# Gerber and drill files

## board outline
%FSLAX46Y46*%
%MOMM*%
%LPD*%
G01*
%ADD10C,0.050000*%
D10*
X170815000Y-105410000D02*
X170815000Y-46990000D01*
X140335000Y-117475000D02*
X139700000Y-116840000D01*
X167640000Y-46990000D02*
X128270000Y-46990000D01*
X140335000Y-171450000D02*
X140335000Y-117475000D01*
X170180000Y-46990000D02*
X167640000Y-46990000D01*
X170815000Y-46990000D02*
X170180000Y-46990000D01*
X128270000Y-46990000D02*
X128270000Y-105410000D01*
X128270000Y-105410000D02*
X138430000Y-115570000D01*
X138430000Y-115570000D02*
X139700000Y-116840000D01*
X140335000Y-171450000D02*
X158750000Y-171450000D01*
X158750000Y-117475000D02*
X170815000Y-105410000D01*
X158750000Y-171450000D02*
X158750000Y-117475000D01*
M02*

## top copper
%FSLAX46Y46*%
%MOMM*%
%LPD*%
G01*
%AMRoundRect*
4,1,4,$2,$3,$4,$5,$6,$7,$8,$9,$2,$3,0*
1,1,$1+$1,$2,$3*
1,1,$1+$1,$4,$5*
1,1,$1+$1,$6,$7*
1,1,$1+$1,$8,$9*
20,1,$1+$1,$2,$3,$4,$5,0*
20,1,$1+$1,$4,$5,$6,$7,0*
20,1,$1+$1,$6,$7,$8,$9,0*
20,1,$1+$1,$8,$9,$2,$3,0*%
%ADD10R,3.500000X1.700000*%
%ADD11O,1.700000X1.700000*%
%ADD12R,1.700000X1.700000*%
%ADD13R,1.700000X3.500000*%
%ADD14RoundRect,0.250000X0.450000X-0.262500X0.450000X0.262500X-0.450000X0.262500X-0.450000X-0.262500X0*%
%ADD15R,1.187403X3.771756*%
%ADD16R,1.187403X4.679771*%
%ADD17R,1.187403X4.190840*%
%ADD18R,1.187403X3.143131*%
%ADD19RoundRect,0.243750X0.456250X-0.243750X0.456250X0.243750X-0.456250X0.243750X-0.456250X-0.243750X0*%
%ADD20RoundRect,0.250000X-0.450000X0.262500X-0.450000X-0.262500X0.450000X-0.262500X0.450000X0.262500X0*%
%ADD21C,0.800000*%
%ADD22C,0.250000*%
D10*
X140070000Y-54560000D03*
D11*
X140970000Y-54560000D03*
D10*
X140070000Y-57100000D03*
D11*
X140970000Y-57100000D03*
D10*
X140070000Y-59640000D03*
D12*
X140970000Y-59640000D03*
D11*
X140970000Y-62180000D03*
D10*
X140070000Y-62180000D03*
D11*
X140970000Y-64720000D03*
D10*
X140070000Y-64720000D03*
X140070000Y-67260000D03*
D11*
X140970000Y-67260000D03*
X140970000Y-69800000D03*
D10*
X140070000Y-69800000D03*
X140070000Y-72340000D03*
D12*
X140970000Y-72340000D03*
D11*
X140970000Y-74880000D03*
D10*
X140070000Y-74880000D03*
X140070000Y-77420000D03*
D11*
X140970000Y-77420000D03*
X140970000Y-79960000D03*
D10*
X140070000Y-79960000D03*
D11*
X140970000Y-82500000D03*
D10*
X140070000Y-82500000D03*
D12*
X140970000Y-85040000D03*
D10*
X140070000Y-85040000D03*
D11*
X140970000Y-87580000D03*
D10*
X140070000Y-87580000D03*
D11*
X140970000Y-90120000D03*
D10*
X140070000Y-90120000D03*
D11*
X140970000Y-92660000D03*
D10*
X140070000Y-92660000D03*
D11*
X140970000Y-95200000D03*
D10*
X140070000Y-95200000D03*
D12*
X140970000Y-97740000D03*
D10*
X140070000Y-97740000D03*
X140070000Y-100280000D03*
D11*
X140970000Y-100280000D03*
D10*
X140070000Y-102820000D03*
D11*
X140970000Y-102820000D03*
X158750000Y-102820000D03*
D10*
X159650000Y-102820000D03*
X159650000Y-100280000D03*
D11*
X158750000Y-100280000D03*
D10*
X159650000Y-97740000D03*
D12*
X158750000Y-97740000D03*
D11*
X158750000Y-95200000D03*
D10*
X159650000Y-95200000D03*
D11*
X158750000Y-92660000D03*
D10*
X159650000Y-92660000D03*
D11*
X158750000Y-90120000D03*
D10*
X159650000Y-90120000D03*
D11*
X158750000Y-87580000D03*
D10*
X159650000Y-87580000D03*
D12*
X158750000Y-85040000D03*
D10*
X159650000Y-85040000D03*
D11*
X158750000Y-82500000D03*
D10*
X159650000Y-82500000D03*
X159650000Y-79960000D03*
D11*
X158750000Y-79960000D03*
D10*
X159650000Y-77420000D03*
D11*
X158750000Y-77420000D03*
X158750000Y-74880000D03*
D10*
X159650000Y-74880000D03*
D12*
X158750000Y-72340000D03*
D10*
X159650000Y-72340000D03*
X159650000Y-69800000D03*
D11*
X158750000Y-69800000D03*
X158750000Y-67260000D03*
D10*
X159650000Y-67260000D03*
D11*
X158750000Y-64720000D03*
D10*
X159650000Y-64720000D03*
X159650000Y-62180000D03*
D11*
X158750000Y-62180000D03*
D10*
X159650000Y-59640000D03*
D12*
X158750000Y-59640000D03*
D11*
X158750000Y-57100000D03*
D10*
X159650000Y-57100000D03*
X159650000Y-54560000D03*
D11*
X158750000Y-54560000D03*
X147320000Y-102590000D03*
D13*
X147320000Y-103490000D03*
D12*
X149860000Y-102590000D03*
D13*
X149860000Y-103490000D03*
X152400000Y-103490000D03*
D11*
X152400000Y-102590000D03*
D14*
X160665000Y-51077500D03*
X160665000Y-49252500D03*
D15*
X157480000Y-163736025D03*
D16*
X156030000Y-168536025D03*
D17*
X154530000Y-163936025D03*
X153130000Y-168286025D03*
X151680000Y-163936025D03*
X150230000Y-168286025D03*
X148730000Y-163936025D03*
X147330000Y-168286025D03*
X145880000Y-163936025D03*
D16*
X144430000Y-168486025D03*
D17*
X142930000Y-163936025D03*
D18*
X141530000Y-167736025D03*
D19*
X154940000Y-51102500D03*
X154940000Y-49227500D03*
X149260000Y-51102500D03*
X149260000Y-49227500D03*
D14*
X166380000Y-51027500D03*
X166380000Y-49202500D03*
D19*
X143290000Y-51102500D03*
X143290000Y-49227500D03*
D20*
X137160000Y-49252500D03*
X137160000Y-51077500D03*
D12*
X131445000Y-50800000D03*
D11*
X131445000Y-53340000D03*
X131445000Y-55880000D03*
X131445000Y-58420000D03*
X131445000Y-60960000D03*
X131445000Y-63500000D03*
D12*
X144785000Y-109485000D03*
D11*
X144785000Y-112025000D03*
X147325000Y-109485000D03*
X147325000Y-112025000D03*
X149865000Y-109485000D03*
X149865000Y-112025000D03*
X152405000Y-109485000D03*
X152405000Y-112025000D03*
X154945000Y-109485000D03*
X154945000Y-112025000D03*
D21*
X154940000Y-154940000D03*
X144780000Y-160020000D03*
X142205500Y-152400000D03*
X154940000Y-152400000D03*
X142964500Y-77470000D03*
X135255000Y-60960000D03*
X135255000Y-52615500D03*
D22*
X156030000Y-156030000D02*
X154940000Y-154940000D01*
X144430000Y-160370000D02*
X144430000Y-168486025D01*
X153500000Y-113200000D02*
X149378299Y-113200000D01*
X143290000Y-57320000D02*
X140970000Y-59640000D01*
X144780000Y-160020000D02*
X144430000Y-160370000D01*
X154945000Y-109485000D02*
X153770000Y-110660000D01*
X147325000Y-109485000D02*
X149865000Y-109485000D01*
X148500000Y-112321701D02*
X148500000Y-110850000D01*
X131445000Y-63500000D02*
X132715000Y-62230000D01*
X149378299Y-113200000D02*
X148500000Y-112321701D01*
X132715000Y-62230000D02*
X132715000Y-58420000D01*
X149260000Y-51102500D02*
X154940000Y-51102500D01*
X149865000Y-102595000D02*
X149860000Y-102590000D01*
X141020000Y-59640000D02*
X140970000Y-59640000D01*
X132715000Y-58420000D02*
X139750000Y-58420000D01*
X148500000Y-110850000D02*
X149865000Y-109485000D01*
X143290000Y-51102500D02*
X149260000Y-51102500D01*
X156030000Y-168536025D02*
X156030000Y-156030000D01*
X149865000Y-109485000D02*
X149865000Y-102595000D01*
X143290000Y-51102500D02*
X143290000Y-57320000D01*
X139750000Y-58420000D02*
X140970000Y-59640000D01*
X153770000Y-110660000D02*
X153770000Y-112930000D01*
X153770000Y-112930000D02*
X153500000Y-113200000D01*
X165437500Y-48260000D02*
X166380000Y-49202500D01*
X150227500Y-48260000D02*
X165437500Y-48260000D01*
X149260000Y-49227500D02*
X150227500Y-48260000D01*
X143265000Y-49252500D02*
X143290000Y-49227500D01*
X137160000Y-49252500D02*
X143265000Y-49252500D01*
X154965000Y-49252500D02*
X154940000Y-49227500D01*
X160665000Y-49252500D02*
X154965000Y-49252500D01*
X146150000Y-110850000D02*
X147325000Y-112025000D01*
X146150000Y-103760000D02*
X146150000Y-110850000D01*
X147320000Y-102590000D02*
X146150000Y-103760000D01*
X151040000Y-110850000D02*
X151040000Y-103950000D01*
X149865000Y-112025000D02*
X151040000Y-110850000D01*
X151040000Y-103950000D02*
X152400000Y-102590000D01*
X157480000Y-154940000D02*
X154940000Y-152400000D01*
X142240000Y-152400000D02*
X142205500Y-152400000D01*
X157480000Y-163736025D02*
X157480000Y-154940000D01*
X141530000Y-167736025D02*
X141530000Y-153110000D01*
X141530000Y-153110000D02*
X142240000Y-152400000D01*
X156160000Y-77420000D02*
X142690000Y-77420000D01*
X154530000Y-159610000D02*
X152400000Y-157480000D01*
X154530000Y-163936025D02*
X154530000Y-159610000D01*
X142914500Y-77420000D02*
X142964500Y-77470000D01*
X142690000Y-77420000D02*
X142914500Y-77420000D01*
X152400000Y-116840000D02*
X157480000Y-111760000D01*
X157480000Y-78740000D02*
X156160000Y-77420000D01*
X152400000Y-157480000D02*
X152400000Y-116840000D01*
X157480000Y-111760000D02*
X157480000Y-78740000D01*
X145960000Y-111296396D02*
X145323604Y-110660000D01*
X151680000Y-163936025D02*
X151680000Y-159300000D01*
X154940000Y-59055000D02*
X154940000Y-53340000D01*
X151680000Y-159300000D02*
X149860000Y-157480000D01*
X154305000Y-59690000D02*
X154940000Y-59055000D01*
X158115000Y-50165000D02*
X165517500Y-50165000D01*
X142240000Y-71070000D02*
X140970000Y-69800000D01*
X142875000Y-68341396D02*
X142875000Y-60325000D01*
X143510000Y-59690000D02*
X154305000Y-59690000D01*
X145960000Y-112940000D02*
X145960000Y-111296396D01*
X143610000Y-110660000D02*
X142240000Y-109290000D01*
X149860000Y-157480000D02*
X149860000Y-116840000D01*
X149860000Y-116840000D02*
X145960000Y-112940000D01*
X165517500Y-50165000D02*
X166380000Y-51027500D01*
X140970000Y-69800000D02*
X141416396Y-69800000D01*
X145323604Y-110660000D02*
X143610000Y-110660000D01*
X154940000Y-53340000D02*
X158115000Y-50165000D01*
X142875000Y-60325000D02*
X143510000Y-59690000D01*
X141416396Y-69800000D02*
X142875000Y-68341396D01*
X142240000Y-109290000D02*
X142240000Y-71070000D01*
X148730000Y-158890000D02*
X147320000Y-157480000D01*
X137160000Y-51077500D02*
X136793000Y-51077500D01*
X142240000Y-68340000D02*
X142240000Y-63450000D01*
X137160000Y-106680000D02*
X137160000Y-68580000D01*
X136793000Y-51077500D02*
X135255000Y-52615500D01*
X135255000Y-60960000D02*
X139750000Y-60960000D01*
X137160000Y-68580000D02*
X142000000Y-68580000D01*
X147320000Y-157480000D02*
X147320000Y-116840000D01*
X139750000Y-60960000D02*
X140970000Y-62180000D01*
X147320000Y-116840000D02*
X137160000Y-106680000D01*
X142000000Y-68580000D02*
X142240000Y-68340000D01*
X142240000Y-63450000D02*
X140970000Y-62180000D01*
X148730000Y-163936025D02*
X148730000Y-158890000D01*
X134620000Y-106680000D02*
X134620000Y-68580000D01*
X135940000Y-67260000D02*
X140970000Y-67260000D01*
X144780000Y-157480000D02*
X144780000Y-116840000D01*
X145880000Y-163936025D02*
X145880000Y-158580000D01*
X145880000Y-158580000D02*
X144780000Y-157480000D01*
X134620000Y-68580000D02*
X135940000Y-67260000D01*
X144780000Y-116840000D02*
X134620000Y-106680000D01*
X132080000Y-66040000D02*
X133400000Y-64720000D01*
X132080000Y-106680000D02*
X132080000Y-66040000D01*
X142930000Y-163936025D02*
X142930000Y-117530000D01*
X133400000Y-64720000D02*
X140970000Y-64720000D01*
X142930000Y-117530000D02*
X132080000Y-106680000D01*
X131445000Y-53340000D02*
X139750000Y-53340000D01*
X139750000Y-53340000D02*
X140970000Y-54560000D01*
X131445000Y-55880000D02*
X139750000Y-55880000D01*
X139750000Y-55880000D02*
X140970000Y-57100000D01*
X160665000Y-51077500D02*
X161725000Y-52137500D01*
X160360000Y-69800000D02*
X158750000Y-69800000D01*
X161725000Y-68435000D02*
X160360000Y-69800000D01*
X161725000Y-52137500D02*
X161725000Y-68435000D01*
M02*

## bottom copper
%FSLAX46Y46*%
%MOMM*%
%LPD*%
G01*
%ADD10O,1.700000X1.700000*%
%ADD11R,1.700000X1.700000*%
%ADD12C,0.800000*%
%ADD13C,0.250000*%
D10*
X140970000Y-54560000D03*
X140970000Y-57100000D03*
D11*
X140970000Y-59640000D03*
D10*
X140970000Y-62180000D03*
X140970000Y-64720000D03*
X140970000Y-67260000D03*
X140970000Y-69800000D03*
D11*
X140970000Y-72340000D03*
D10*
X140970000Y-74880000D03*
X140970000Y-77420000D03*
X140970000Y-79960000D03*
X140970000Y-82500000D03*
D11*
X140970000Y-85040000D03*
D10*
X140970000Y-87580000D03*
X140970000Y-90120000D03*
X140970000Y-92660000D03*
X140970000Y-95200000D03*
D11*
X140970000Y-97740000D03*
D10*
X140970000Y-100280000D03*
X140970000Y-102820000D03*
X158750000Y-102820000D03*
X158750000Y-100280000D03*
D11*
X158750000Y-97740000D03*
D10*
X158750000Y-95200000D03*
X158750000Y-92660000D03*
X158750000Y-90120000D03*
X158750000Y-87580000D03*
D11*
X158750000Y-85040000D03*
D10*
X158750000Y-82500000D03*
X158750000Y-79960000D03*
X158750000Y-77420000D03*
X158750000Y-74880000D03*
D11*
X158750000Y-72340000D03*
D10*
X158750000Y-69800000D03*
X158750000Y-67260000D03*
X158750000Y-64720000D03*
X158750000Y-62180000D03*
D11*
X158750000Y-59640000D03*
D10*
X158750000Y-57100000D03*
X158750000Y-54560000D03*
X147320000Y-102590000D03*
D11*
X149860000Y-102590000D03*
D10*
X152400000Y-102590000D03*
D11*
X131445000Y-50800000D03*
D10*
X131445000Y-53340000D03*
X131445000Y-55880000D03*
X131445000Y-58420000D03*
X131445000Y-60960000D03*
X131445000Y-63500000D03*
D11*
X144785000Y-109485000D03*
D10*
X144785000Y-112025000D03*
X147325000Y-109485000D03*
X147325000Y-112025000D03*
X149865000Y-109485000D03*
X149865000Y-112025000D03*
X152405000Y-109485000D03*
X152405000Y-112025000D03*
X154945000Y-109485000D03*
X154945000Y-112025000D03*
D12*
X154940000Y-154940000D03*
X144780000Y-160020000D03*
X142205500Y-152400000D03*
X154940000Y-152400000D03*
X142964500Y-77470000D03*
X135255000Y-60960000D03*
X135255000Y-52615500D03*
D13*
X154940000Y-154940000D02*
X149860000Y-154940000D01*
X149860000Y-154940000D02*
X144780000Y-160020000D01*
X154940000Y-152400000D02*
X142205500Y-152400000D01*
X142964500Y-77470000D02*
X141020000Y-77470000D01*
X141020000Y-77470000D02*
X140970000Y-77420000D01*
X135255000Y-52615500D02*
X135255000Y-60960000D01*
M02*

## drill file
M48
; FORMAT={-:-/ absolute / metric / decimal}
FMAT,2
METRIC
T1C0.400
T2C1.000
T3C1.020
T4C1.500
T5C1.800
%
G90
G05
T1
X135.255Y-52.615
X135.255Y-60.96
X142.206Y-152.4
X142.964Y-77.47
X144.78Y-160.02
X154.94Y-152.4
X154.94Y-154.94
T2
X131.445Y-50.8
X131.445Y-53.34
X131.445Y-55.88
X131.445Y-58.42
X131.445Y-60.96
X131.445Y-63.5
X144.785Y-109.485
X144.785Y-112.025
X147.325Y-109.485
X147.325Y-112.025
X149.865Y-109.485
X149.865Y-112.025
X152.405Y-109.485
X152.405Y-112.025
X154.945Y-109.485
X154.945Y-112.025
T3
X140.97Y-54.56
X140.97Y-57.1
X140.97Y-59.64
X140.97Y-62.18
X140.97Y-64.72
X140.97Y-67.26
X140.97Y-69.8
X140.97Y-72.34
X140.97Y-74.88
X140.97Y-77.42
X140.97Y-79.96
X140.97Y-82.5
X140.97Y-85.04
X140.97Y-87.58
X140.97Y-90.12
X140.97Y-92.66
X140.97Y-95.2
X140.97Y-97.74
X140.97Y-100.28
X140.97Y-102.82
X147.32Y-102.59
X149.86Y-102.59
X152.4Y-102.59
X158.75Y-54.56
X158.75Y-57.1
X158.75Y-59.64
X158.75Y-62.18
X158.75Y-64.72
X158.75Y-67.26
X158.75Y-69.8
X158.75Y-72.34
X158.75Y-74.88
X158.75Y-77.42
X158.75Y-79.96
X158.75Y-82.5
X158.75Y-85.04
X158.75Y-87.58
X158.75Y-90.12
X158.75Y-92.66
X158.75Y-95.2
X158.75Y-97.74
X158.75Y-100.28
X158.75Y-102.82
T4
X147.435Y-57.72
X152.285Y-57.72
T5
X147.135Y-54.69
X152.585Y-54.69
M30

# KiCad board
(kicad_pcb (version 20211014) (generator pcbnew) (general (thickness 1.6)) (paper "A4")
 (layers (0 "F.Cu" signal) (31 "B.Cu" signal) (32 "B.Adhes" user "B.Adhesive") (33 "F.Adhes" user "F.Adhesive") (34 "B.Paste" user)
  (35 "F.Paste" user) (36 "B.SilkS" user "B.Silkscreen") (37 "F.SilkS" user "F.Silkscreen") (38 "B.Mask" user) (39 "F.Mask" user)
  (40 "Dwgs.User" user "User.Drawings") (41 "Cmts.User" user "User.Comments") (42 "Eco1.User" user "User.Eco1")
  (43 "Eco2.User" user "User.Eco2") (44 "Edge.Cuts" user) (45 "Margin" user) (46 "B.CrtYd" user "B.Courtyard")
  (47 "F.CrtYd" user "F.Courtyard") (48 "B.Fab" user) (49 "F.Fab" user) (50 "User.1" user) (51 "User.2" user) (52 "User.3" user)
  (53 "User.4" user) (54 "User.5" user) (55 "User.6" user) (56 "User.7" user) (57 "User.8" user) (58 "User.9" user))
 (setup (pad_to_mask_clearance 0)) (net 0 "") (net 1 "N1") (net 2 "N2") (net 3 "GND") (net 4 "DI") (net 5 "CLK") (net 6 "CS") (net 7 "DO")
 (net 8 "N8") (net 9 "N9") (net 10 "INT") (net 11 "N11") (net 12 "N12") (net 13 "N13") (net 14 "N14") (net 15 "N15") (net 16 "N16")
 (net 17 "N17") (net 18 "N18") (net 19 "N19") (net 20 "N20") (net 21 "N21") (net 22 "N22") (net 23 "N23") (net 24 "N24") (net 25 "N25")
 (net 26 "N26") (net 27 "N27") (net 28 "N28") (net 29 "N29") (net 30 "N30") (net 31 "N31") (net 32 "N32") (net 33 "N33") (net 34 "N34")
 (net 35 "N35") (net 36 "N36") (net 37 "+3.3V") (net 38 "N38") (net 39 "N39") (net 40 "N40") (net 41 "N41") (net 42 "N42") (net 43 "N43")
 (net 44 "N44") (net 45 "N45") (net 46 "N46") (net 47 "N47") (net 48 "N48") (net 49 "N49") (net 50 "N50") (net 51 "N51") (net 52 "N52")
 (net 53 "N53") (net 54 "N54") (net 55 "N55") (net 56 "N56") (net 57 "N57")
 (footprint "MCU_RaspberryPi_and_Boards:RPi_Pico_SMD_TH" (layer "F.Cu") (at 149.86 78.69)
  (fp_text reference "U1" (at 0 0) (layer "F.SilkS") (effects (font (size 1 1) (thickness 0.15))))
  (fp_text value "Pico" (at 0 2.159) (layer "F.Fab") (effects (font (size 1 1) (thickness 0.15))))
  (pad "" np_thru_hole oval (at -2.725 -24) (size 1.8 1.8) (drill 1.8) (layers *.Cu *.Mask))
  (pad "" np_thru_hole oval (at 2.725 -24) (size 1.8 1.8) (drill 1.8) (layers *.Cu *.Mask))
  (pad "" np_thru_hole oval (at 2.425 -20.97) (size 1.5 1.5) (drill 1.5) (layers *.Cu *.Mask))
  (pad "" np_thru_hole oval (at -2.425 -20.97) (size 1.5 1.5) (drill 1.5) (layers *.Cu *.Mask))
  (pad "1" smd rect (at -8.89 -24.13) (size 3.5 1.7) (drill (offset -0.9 0)) (layers "F.Cu" "F.Mask") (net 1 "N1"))
  (pad "1" thru_hole oval (at -8.89 -24.13) (size 1.7 1.7) (drill 1.02) (layers *.Cu *.Mask) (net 1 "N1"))
  (pad "2" smd rect (at -8.89 -21.59) (size 3.5 1.7) (drill (offset -0.9 0)) (layers "F.Cu" "F.Mask") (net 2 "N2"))
  (pad "2" thru_hole oval (at -8.89 -21.59) (size 1.7 1.7) (drill 1.02) (layers *.Cu *.Mask) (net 2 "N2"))
  (pad "3" smd rect (at -8.89 -19.05) (size 3.5 1.7) (drill (offset -0.9 0)) (layers "F.Cu" "F.Mask") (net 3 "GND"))
  (pad "3" thru_hole rect (at -8.89 -19.05) (size 1.7 1.7) (drill 1.02) (layers *.Cu *.Mask) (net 3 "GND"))
  (pad "4" thru_hole oval (at -8.89 -16.51) (size 1.7 1.7) (drill 1.02) (layers *.Cu *.Mask) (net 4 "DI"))
  (pad "4" smd rect (at -8.89 -16.51) (size 3.5 1.7) (drill (offset -0.9 0)) (layers "F.Cu" "F.Mask") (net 4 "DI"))
  (pad "5" thru_hole oval (at -8.89 -13.97) (size 1.7 1.7) (drill 1.02) (layers *.Cu *.Mask) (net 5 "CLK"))
  (pad "5" smd rect (at -8.89 -13.97) (size 3.5 1.7) (drill (offset -0.9 0)) (layers "F.Cu" "F.Mask") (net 5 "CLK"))
  (pad "6" smd rect (at -8.89 -11.43) (size 3.5 1.7) (drill (offset -0.9 0)) (layers "F.Cu" "F.Mask") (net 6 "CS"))
  (pad "6" thru_hole oval (at -8.89 -11.43) (size 1.7 1.7) (drill 1.02) (layers *.Cu *.Mask) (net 6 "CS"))
  (pad "7" thru_hole oval (at -8.89 -8.89) (size 1.7 1.7) (drill 1.02) (layers *.Cu *.Mask) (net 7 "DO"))
  (pad "7" smd rect (at -8.89 -8.89) (size 3.5 1.7) (drill (offset -0.9 0)) (layers "F.Cu" "F.Mask") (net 7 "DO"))
  (pad "8" smd rect (at -8.89 -6.35) (size 3.5 1.7) (drill (offset -0.9 0)) (layers "F.Cu" "F.Mask") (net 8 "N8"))
  (pad "8" thru_hole rect (at -8.89 -6.35) (size 1.7 1.7) (drill 1.02) (layers *.Cu *.Mask) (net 8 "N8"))
  (pad "9" thru_hole oval (at -8.89 -3.81) (size 1.7 1.7) (drill 1.02) (layers *.Cu *.Mask) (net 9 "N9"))
  (pad "9" smd rect (at -8.89 -3.81) (size 3.5 1.7) (drill (offset -0.9 0)) (layers "F.Cu" "F.Mask") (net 9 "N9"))
  (pad "10" smd rect (at -8.89 -1.27) (size 3.5 1.7) (drill (offset -0.9 0)) (layers "F.Cu" "F.Mask") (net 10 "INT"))
  (pad "10" thru_hole oval (at -8.89 -1.27) (size 1.7 1.7) (drill 1.02) (layers *.Cu *.Mask) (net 10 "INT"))
  (pad "11" thru_hole oval (at -8.89 1.27) (size 1.7 1.7) (drill 1.02) (layers *.Cu *.Mask) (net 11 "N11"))
  (pad "11" smd rect (at -8.89 1.27) (size 3.5 1.7) (drill (offset -0.9 0)) (layers "F.Cu" "F.Mask") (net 11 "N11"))
  (pad "12" thru_hole oval (at -8.89 3.81) (size 1.7 1.7) (drill 1.02) (layers *.Cu *.Mask) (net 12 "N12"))
  (pad "12" smd rect (at -8.89 3.81) (size 3.5 1.7) (drill (offset -0.9 0)) (layers "F.Cu" "F.Mask") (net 12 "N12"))
  (pad "13" thru_hole rect (at -8.89 6.35) (size 1.7 1.7) (drill 1.02) (layers *.Cu *.Mask) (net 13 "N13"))
  (pad "13" smd rect (at -8.89 6.35) (size 3.5 1.7) (drill (offset -0.9 0)) (layers "F.Cu" "F.Mask") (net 13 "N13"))
  (pad "14" thru_hole oval (at -8.89 8.89) (size 1.7 1.7) (drill 1.02) (layers *.Cu *.Mask) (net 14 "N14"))
  (pad "14" smd rect (at -8.89 8.89) (size 3.5 1.7) (drill (offset -0.9 0)) (layers "F.Cu" "F.Mask") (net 14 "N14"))
  (pad "15" thru_hole oval (at -8.89 11.43) (size 1.7 1.7) (drill 1.02) (layers *.Cu *.Mask) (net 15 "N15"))
  (pad "15" smd rect (at -8.89 11.43) (size 3.5 1.7) (drill (offset -0.9 0)) (layers "F.Cu" "F.Mask") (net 15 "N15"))
  (pad "16" thru_hole oval (at -8.89 13.97) (size 1.7 1.7) (drill 1.02) (layers *.Cu *.Mask) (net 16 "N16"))
  (pad "16" smd rect (at -8.89 13.97) (size 3.5 1.7) (drill (offset -0.9 0)) (layers "F.Cu" "F.Mask") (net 16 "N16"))
  (pad "17" thru_hole oval (at -8.89 16.51) (size 1.7 1.7) (drill 1.02) (layers *.Cu *.Mask) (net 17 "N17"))
  (pad "17" smd rect (at -8.89 16.51) (size 3.5 1.7) (drill (offset -0.9 0)) (layers "F.Cu" "F.Mask") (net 17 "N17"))
  (pad "18" thru_hole rect (at -8.89 19.05) (size 1.7 1.7) (drill 1.02) (layers *.Cu *.Mask) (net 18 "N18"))
  (pad "18" smd rect (at -8.89 19.05) (size 3.5 1.7) (drill (offset -0.9 0)) (layers "F.Cu" "F.Mask") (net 18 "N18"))
  (pad "19" smd rect (at -8.89 21.59) (size 3.5 1.7) (drill (offset -0.9 0)) (layers "F.Cu" "F.Mask") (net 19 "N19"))
  (pad "19" thru_hole oval (at -8.89 21.59) (size 1.7 1.7) (drill 1.02) (layers *.Cu *.Mask) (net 19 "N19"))
  (pad "20" smd rect (at -8.89 24.13) (size 3.5 1.7) (drill (offset -0.9 0)) (layers "F.Cu" "F.Mask") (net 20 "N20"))
  (pad "20" thru_hole oval (at -8.89 24.13) (size 1.7 1.7) (drill 1.02) (layers *.Cu *.Mask) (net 20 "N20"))
  (pad "21" thru_hole oval (at 8.89 24.13) (size 1.7 1.7) (drill 1.02) (layers *.Cu *.Mask) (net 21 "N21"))
  (pad "21" smd rect (at 8.89 24.13) (size 3.5 1.7) (drill (offset 0.9 0)) (layers "F.Cu" "F.Mask") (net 21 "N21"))
  (pad "22" smd rect (at 8.89 21.59) (size 3.5 1.7) (drill (offset 0.9 0)) (layers "F.Cu" "F.Mask") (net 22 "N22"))
  (pad "22" thru_hole oval (at 8.89 21.59) (size 1.7 1.7) (drill 1.02) (layers *.Cu *.Mask) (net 22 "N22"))
  (pad "23" smd rect (at 8.89 19.05) (size 3.5 1.7) (drill (offset 0.9 0)) (layers "F.Cu" "F.Mask") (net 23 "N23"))
  (pad "23" thru_hole rect (at 8.89 19.05) (size 1.7 1.7) (drill 1.02) (layers *.Cu *.Mask) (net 23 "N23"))
  (pad "24" thru_hole oval (at 8.89 16.51) (size 1.7 1.7) (drill 1.02) (layers *.Cu *.Mask) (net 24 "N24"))
  (pad "24" smd rect (at 8.89 16.51) (size 3.5 1.7) (drill (offset 0.9 0)) (layers "F.Cu" "F.Mask") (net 24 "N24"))
  (pad "25" thru_hole oval (at 8.89 13.97) (size 1.7 1.7) (drill 1.02) (layers *.Cu *.Mask) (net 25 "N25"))
  (pad "25" smd rect (at 8.89 13.97) (size 3.5 1.7) (drill (offset 0.9 0)) (layers "F.Cu" "F.Mask") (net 25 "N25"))
  (pad "26" thru_hole oval (at 8.89 11.43) (size 1.7 1.7) (drill 1.02) (layers *.Cu *.Mask) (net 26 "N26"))
  (pad "26" smd rect (at 8.89 11.43) (size 3.5 1.7) (drill (offset 0.9 0)) (layers "F.Cu" "F.Mask") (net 26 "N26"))
  (pad "27" thru_hole oval (at 8.89 8.89) (size 1.7 1.7) (drill 1.02) (layers *.Cu *.Mask) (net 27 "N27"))
  (pad "27" smd rect (at 8.89 8.89) (size 3.5 1.7) (drill (offset 0.9 0)) (layers "F.Cu" "F.Mask") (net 27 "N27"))
  (pad "28" thru_hole rect (at 8.89 6.35) (size 1.7 1.7) (drill 1.02) (layers *.Cu *.Mask) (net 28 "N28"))
  (pad "28" smd rect (at 8.89 6.35) (size 3.5 1.7) (drill (offset 0.9 0)) (layers "F.Cu" "F.Mask") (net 28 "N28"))
  (pad "29" thru_hole oval (at 8.89 3.81) (size 1.7 1.7) (drill 1.02) (layers *.Cu *.Mask) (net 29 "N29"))
  (pad "29" smd rect (at 8.89 3.81) (size 3.5 1.7) (drill (offset 0.9 0)) (layers "F.Cu" "F.Mask") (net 29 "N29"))
  (pad "30" smd rect (at 8.89 1.27) (size 3.5 1.7) (drill (offset 0.9 0)) (layers "F.Cu" "F.Mask") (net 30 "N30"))
  (pad "30" thru_hole oval (at 8.89 1.27) (size 1.7 1.7) (drill 1.02) (layers *.Cu *.Mask) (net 30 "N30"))
  (pad "31" smd rect (at 8.89 -1.27) (size 3.5 1.7) (drill (offset 0.9 0)) (layers "F.Cu" "F.Mask") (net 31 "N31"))
  (pad "31" thru_hole oval (at 8.89 -1.27) (size 1.7 1.7) (drill 1.02) (layers *.Cu *.Mask) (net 31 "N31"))
  (pad "32" thru_hole oval (at 8.89 -3.81) (size 1.7 1.7) (drill 1.02) (layers *.Cu *.Mask) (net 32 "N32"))
  (pad "32" smd rect (at 8.89 -3.81) (size 3.5 1.7) (drill (offset 0.9 0)) (layers "F.Cu" "F.Mask") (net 32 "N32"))
  (pad "33" thru_hole rect (at 8.89 -6.35) (size 1.7 1.7) (drill 1.02) (layers *.Cu *.Mask) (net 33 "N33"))
  (pad "33" smd rect (at 8.89 -6.35) (size 3.5 1.7) (drill (offset 0.9 0)) (layers "F.Cu" "F.Mask") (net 33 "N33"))
  (pad "34" smd rect (at 8.89 -8.89) (size 3.5 1.7) (drill (offset 0.9 0)) (layers "F.Cu" "F.Mask") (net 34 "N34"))
  (pad "34" thru_hole oval (at 8.89 -8.89) (size 1.7 1.7) (drill 1.02) (layers *.Cu *.Mask) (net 34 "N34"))
  (pad "35" thru_hole oval (at 8.89 -11.43) (size 1.7 1.7) (drill 1.02) (layers *.Cu *.Mask) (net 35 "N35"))
  (pad "35" smd rect (at 8.89 -11.43) (size 3.5 1.7) (drill (offset 0.9 0)) (layers "F.Cu" "F.Mask") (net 35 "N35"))
  (pad "36" thru_hole oval (at 8.89 -13.97) (size 1.7 1.7) (drill 1.02) (layers *.Cu *.Mask) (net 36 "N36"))
  (pad "36" smd rect (at 8.89 -13.97) (size 3.5 1.7) (drill (offset 0.9 0)) (layers "F.Cu" "F.Mask") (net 36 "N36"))
  (pad "37" smd rect (at 8.89 -16.51) (size 3.5 1.7) (drill (offset 0.9 0)) (layers "F.Cu" "F.Mask") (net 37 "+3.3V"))
  (pad "37" thru_hole oval (at 8.89 -16.51) (size 1.7 1.7) (drill 1.02) (layers *.Cu *.Mask) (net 37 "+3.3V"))
  (pad "38" smd rect (at 8.89 -19.05) (size 3.5 1.7) (drill (offset 0.9 0)) (layers "F.Cu" "F.Mask") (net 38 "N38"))
  (pad "38" thru_hole rect (at 8.89 -19.05) (size 1.7 1.7) (drill 1.02) (layers *.Cu *.Mask) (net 38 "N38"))
  (pad "39" thru_hole oval (at 8.89 -21.59) (size 1.7 1.7) (drill 1.02) (layers *.Cu *.Mask) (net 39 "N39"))
  (pad "39" smd rect (at 8.89 -21.59) (size 3.5 1.7) (drill (offset 0.9 0)) (layers "F.Cu" "F.Mask") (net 39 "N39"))
  (pad "40" smd rect (at 8.89 -24.13) (size 3.5 1.7) (drill (offset 0.9 0)) (layers "F.Cu" "F.Mask") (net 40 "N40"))
  (pad "40" thru_hole oval (at 8.89 -24.13) (size 1.7 1.7) (drill 1.02) (layers *.Cu *.Mask) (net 40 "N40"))
  (pad "41" thru_hole oval (at -2.54 23.9) (size 1.7 1.7) (drill 1.02) (layers *.Cu *.Mask) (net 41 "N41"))
  (pad "41" smd rect (at -2.54 23.9 90) (size 3.5 1.7) (drill (offset -0.9 0)) (layers "F.Cu" "F.Mask") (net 41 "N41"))
  (pad "42" thru_hole rect (at 0 23.9) (size 1.7 1.7) (drill 1.02) (layers *.Cu *.Mask) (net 3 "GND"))
  (pad "42" smd rect (at 0 23.9 90) (size 3.5 1.7) (drill (offset -0.9 0)) (layers "F.Cu" "F.Mask") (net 3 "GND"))
  (pad "43" smd rect (at 2.54 23.9 90) (size 3.5 1.7) (drill (offset -0.9 0)) (layers "F.Cu" "F.Mask") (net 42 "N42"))
  (pad "43" thru_hole oval (at 2.54 23.9) (size 1.7 1.7) (drill 1.02) (layers *.Cu *.Mask) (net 42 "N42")))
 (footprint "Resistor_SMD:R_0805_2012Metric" (layer "F.Cu") (at 160.665 50.165 90)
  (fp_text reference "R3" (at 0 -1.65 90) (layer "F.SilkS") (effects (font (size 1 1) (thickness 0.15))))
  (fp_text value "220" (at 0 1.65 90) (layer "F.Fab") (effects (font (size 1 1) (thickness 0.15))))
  (pad "1" smd roundrect (at -0.9125 0 90) (size 1.025 1.4) (layers "F.Cu" "F.Paste" "F.Mask") (roundrect_rratio 0.243902439) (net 34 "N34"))
  (pad "2" smd roundrect (at 0.9125 0 90) (size 1.025 1.4) (layers "F.Cu" "F.Paste" "F.Mask") (roundrect_rratio 0.243902439) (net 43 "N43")))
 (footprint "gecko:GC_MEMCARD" (layer "F.Cu") (at 140.43 171.316025)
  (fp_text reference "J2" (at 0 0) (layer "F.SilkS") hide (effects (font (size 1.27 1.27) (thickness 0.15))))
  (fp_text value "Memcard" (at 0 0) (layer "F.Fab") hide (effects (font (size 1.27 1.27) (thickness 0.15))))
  (pad "1" smd rect (at 17.05 -7.58) (size 1.187403 3.771756) (layers "F.Cu" "F.Paste" "F.Mask") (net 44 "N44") (solder_mask_margin 0.0762))
  (pad "2" smd rect (at 15.6 -2.78) (size 1.187403 4.679771) (layers "F.Cu" "F.Paste" "F.Mask") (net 3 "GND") (solder_mask_margin 0.0762))
  (pad "3" smd rect (at 14.1 -7.38) (size 1.187403 4.19084) (layers "F.Cu" "F.Paste" "F.Mask") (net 10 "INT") (solder_mask_margin 0.0762))
  (pad "4" smd rect (at 12.7 -3.03) (size 1.187403 4.19084) (layers "F.Cu" "F.Paste" "F.Mask") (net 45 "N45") (solder_mask_margin 0.0762))
  (pad "5" smd rect (at 11.25 -7.38) (size 1.187403 4.19084) (layers "F.Cu" "F.Paste" "F.Mask") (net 7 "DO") (solder_mask_margin 0.0762))
  (pad "6" smd rect (at 9.8 -3.03) (size 1.187403 4.19084) (layers "F.Cu" "F.Paste" "F.Mask") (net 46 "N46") (solder_mask_margin 0.0762))
  (pad "7" smd rect (at 8.3 -7.38) (size 1.187403 4.19084) (layers "F.Cu" "F.Paste" "F.Mask") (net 4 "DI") (solder_mask_margin 0.0762))
  (pad "8" smd rect (at 6.9 -3.03) (size 1.187403 4.19084) (layers "F.Cu" "F.Paste" "F.Mask") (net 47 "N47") (solder_mask_margin 0.0762))
  (pad "9" smd rect (at 5.45 -7.38) (size 1.187403 4.19084) (layers "F.Cu" "F.Paste" "F.Mask") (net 6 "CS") (solder_mask_margin 0.0762))
  (pad "10" smd rect (at 4 -2.83) (size 1.187403 4.679771) (layers "F.Cu" "F.Paste" "F.Mask") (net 3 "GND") (solder_mask_margin 0.0762))
  (pad "11" smd rect (at 2.5 -7.38) (size 1.187403 4.19084) (layers "F.Cu" "F.Paste" "F.Mask") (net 5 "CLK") (solder_mask_margin 0.0762))
  (pad "12" smd rect (at 1.1 -3.58) (size 1.187403 3.143131) (layers "F.Cu" "F.Paste" "F.Mask") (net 44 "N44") (solder_mask_margin 0.0762)))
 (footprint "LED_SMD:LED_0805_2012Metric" (layer "F.Cu") (at 154.94 50.165 90)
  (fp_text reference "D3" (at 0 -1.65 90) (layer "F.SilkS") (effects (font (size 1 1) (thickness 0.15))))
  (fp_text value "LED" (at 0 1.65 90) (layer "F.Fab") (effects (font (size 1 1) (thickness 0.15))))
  (pad "1" smd roundrect (at -0.9375 0 90) (size 0.975 1.4) (layers "F.Cu" "F.Paste" "F.Mask") (roundrect_rratio 0.25) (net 3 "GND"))
  (pad "2" smd roundrect (at 0.9375 0 90) (size 0.975 1.4) (layers "F.Cu" "F.Paste" "F.Mask") (roundrect_rratio 0.25) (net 43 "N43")))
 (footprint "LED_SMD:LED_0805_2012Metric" (layer "F.Cu") (at 149.26 50.165 90)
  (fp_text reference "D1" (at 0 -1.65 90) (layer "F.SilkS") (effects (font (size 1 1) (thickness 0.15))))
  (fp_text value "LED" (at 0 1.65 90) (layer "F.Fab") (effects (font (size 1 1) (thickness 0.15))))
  (pad "1" smd roundrect (at -0.9375 0 90) (size 0.975 1.4) (layers "F.Cu" "F.Paste" "F.Mask") (roundrect_rratio 0.25) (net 3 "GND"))
  (pad "2" smd roundrect (at 0.9375 0 90) (size 0.975 1.4) (layers "F.Cu" "F.Paste" "F.Mask") (roundrect_rratio 0.25) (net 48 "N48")))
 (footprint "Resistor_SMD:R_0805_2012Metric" (layer "F.Cu") (at 166.38 50.115 90)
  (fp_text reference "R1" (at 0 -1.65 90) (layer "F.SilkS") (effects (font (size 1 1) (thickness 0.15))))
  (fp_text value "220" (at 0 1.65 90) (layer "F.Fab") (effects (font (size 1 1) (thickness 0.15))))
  (pad "1" smd roundrect (at -0.9125 0 90) (size 1.025 1.4) (layers "F.Cu" "F.Paste" "F.Mask") (roundrect_rratio 0.243902439) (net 7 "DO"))
  (pad "2" smd roundrect (at 0.9125 0 90) (size 1.025 1.4) (layers "F.Cu" "F.Paste" "F.Mask") (roundrect_rratio 0.243902439) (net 48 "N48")))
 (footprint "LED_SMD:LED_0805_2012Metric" (layer "F.Cu") (at 143.29 50.165 90)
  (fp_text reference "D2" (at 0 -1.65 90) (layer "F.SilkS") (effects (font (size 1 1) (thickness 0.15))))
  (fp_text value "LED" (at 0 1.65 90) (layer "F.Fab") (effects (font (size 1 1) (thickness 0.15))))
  (pad "1" smd roundrect (at -0.9375 0 90) (size 0.975 1.4) (layers "F.Cu" "F.Paste" "F.Mask") (roundrect_rratio 0.25) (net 3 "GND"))
  (pad "2" smd roundrect (at 0.9375 0 90) (size 0.975 1.4) (layers "F.Cu" "F.Paste" "F.Mask") (roundrect_rratio 0.25) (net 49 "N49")))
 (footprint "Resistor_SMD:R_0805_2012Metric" (layer "F.Cu") (at 137.16 50.165 -90)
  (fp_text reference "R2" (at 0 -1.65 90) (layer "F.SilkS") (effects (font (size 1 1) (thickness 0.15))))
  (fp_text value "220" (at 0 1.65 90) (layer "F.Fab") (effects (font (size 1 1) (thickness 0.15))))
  (pad "1" smd roundrect (at -0.9125 0 270) (size 1.025 1.4) (layers "F.Cu" "F.Paste" "F.Mask") (roundrect_rratio 0.243902439)
   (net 49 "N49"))
  (pad "2" smd roundrect (at 0.9125 0 270) (size 1.025 1.4) (layers "F.Cu" "F.Paste" "F.Mask") (roundrect_rratio 0.243902439) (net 4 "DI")))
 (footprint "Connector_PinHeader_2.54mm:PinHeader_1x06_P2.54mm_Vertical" (layer "B.Cu") (at 131.445 50.8 180)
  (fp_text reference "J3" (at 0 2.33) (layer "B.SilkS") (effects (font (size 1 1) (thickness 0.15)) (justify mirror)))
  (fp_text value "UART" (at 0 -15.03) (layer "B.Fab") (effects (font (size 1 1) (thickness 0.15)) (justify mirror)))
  (pad "1" thru_hole rect (at 0 0 180) (size 1.7 1.7) (drill 1) (layers *.Cu *.Mask) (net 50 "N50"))
  (pad "2" thru_hole oval (at 0 -2.54 180) (size 1.7 1.7) (drill 1) (layers *.Cu *.Mask) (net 1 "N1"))
  (pad "3" thru_hole oval (at 0 -5.08 180) (size 1.7 1.7) (drill 1) (layers *.Cu *.Mask) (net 2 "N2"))
  (pad "4" thru_hole oval (at 0 -7.62 180) (size 1.7 1.7) (drill 1) (layers *.Cu *.Mask) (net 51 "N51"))
  (pad "5" thru_hole oval (at 0 -10.16 180) (size 1.7 1.7) (drill 1) (layers *.Cu *.Mask) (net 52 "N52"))
  (pad "6" thru_hole oval (at 0 -12.7 180) (size 1.7 1.7) (drill 1) (layers *.Cu *.Mask) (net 3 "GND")))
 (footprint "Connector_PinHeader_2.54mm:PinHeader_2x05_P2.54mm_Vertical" (layer "B.Cu") (at 144.785 109.485 -90)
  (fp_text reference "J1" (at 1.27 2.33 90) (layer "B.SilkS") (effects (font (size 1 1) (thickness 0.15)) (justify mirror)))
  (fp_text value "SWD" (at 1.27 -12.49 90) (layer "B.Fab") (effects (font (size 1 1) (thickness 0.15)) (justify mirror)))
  (pad "1" thru_hole rect (at 0 0 270) (size 1.7 1.7) (drill 1) (layers *.Cu *.Mask) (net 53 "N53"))
  (pad "2" thru_hole oval (at 2.54 0 270) (size 1.7 1.7) (drill 1) (layers *.Cu *.Mask) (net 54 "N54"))
  (pad "3" thru_hole oval (at 0 -2.54 270) (size 1.7 1.7) (drill 1) (layers *.Cu *.Mask) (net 3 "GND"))
  (pad "4" thru_hole oval (at 2.54 -2.54 270) (size 1.7 1.7) (drill 1) (layers *.Cu *.Mask) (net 41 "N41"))
  (pad "5" thru_hole oval (at 0 -5.08 270) (size 1.7 1.7) (drill 1) (layers *.Cu *.Mask) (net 3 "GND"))
  (pad "6" thru_hole oval (at 2.54 -5.08 270) (size 1.7 1.7) (drill 1) (layers *.Cu *.Mask) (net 42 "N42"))
  (pad "7" thru_hole oval (at 0 -7.62 270) (size 1.7 1.7) (drill 1) (layers *.Cu *.Mask) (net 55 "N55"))
  (pad "8" thru_hole oval (at 2.54 -7.62 270) (size 1.7 1.7) (drill 1) (layers *.Cu *.Mask) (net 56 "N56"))
  (pad "9" thru_hole oval (at 0 -10.16 270) (size 1.7 1.7) (drill 1) (layers *.Cu *.Mask) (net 3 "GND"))
  (pad "10" thru_hole oval (at 2.54 -10.16 270) (size 1.7 1.7) (drill 1) (layers *.Cu *.Mask) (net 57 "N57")))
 (gr_line (start 170.815 105.41) (end 170.815 46.99) (layer "Edge.Cuts") (width 0.05))
 (gr_line (start 140.335 117.475) (end 139.7 116.84) (layer "Edge.Cuts") (width 0.05))
 (gr_line (start 167.64 46.99) (end 128.27 46.99) (layer "Edge.Cuts") (width 0.05))
 (gr_line (start 140.335 171.45) (end 140.335 117.475) (layer "Edge.Cuts") (width 0.05))
 (gr_line (start 170.18 46.99) (end 167.64 46.99) (layer "Edge.Cuts") (width 0.05))
 (gr_line (start 170.815 46.99) (end 170.18 46.99) (layer "Edge.Cuts") (width 0.05))
 (gr_line (start 128.27 46.99) (end 128.27 105.41) (layer "Edge.Cuts") (width 0.05))
 (gr_line (start 128.27 105.41) (end 138.43 115.57) (layer "Edge.Cuts") (width 0.05))
 (gr_line (start 138.43 115.57) (end 139.7 116.84) (layer "Edge.Cuts") (width 0.05))
 (gr_line (start 140.335 171.45) (end 158.75 171.45) (layer "Edge.Cuts") (width 0.05))
 (gr_line (start 158.75 117.475) (end 170.815 105.41) (layer "Edge.Cuts") (width 0.05))
 (gr_line (start 158.75 171.45) (end 158.75 117.475) (layer "Edge.Cuts") (width 0.05))
 (segment (start 156.03 156.03) (end 154.94 154.94) (width 0.25) (layer "F.Cu") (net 3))
 (segment (start 144.43 160.37) (end 144.43 168.486025) (width 0.25) (layer "F.Cu") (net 3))
 (segment (start 153.5 113.2) (end 149.378299 113.2) (width 0.25) (layer "F.Cu") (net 3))
 (segment (start 143.29 57.32) (end 140.97 59.64) (width 0.25) (layer "F.Cu") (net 3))
 (segment (start 144.78 160.02) (end 144.43 160.37) (width 0.25) (layer "F.Cu") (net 3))
 (segment (start 154.945 109.485) (end 153.77 110.66) (width 0.25) (layer "F.Cu") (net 3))
 (segment (start 147.325 109.485) (end 149.865 109.485) (width 0.25) (layer "F.Cu") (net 3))
 (segment (start 148.5 112.321701) (end 148.5 110.85) (width 0.25) (layer "F.Cu") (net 3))
 (segment (start 131.445 63.5) (end 132.715 62.23) (width 0.25) (layer "F.Cu") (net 3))
 (segment (start 149.378299 113.2) (end 148.5 112.321701) (width 0.25) (layer "F.Cu") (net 3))
 (segment (start 132.715 62.23) (end 132.715 58.42) (width 0.25) (layer "F.Cu") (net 3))
 (segment (start 149.26 51.1025) (end 154.94 51.1025) (width 0.25) (layer "F.Cu") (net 3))
 (segment (start 149.865 102.595) (end 149.86 102.59) (width 0.25) (layer "F.Cu") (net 3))
 (segment (start 141.02 59.64) (end 140.97 59.64) (width 0.25) (layer "F.Cu") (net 3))
 (segment (start 132.715 58.42) (end 139.75 58.42) (width 0.25) (layer "F.Cu") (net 3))
 (segment (start 148.5 110.85) (end 149.865 109.485) (width 0.25) (layer "F.Cu") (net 3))
 (segment (start 143.29 51.1025) (end 149.26 51.1025) (width 0.25) (layer "F.Cu") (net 3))
 (segment (start 156.03 168.536025) (end 156.03 156.03) (width 0.25) (layer "F.Cu") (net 3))
 (segment (start 149.865 109.485) (end 149.865 102.595) (width 0.25) (layer "F.Cu") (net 3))
 (segment (start 143.29 51.1025) (end 143.29 57.32) (width 0.25) (layer "F.Cu") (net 3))
 (segment (start 139.75 58.42) (end 140.97 59.64) (width 0.25) (layer "F.Cu") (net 3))
 (segment (start 153.77 110.66) (end 153.77 112.93) (width 0.25) (layer "F.Cu") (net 3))
 (segment (start 153.77 112.93) (end 153.5 113.2) (width 0.25) (layer "F.Cu") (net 3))
 (via (at 154.94 154.94) (size 0.8) (drill 0.4) (layers "F.Cu" "B.Cu") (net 3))
 (via (at 144.78 160.02) (size 0.8) (drill 0.4) (layers "F.Cu" "B.Cu") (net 3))
 (segment (start 154.94 154.94) (end 149.86 154.94) (width 0.25) (layer "B.Cu") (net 3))
 (segment (start 149.86 154.94) (end 144.78 160.02) (width 0.25) (layer "B.Cu") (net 3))
 (segment (start 165.4375 48.26) (end 166.38 49.2025) (width 0.25) (layer "F.Cu") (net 48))
 (segment (start 150.2275 48.26) (end 165.4375 48.26) (width 0.25) (layer "F.Cu") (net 48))
 (segment (start 149.26 49.2275) (end 150.2275 48.26) (width 0.25) (layer "F.Cu") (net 48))
 (segment (start 143.265 49.2525) (end 143.29 49.2275) (width 0.25) (layer "F.Cu") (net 49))
 (segment (start 137.16 49.2525) (end 143.265 49.2525) (width 0.25) (layer "F.Cu") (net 49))
 (segment (start 154.965 49.2525) (end 154.94 49.2275) (width 0.25) (layer "F.Cu") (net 43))
 (segment (start 160.665 49.2525) (end 154.965 49.2525) (width 0.25) (layer "F.Cu") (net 43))
 (segment (start 146.15 110.85) (end 147.325 112.025) (width 0.25) (layer "F.Cu") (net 41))
 (segment (start 146.15 103.76) (end 146.15 110.85) (width 0.25) (layer "F.Cu") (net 41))
 (segment (start 147.32 102.59) (end 146.15 103.76) (width 0.25) (layer "F.Cu") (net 41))
 (segment (start 151.04 110.85) (end 151.04 103.95) (width 0.25) (layer "F.Cu") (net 42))
 (segment (start 149.865 112.025) (end 151.04 110.85) (width 0.25) (layer "F.Cu") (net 42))
 (segment (start 151.04 103.95) (end 152.4 102.59) (width 0.25) (layer "F.Cu") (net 42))
 (segment (start 157.48 154.94) (end 154.94 152.4) (width 0.25) (layer "F.Cu") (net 44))
 (segment (start 142.24 152.4) (end 142.2055 152.4) (width 0.25) (layer "F.Cu") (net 44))
 (segment (start 157.48 163.736025) (end 157.48 154.94) (width 0.25) (layer "F.Cu") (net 44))
 (segment (start 141.53 167.736025) (end 141.53 153.11) (width 0.25) (layer "F.Cu") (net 44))
 (segment (start 141.53 153.11) (end 142.24 152.4) (width 0.25) (layer "F.Cu") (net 44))
 (via (at 142.2055 152.4) (size 0.8) (drill 0.4) (layers "F.Cu" "B.Cu") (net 44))
 (via (at 154.94 152.4) (size 0.8) (drill 0.4) (layers "F.Cu" "B.Cu") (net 44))
 (segment (start 154.94 152.4) (end 142.2055 152.4) (width 0.25) (layer "B.Cu") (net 44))
 (segment (start 156.16 77.42) (end 142.69 77.42) (width 0.25) (layer "F.Cu") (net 10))
 (segment (start 154.53 159.61) (end 152.4 157.48) (width 0.25) (layer "F.Cu") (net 10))
 (segment (start 154.53 163.936025) (end 154.53 159.61) (width 0.25) (layer "F.Cu") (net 10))
 (segment (start 142.9145 77.42) (end 142.9645 77.47) (width 0.25) (layer "F.Cu") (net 10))
 (segment (start 142.69 77.42) (end 142.9145 77.42) (width 0.25) (layer "F.Cu") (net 10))
 (segment (start 152.4 116.84) (end 157.48 111.76) (width 0.25) (layer "F.Cu") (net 10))
 (segment (start 157.48 78.74) (end 156.16 77.42) (width 0.25) (layer "F.Cu") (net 10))
 (segment (start 152.4 157.48) (end 152.4 116.84) (width 0.25) (layer "F.Cu") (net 10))
 (segment (start 157.48 111.76) (end 157.48 78.74) (width 0.25) (layer "F.Cu") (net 10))
 (via (at 142.9645 77.47) (size 0.8) (drill 0.4) (layers "F.Cu" "B.Cu") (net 10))
 (segment (start 142.9645 77.47) (end 141.02 77.47) (width 0.25) (layer "B.Cu") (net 10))
 (segment (start 141.02 77.47) (end 140.97 77.42) (width 0.25) (layer "B.Cu") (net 10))
 (segment (start 145.96 111.296396) (end 145.323604 110.66) (width 0.25) (layer "F.Cu") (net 7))
 (segment (start 151.68 163.936025) (end 151.68 159.3) (width 0.25) (layer "F.Cu") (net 7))
 (segment (start 154.94 59.055) (end 154.94 53.34) (width 0.25) (layer "F.Cu") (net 7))
 (segment (start 151.68 159.3) (end 149.86 157.48) (width 0.25) (layer "F.Cu") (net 7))
 (segment (start 154.305 59.69) (end 154.94 59.055) (width 0.25) (layer "F.Cu") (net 7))
 (segment (start 158.115 50.165) (end 165.5175 50.165) (width 0.25) (layer "F.Cu") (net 7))
 (segment (start 142.24 71.07) (end 140.97 69.8) (width 0.25) (layer "F.Cu") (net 7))
 (segment (start 142.875 68.341396) (end 142.875 60.325) (width 0.25) (layer "F.Cu") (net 7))
 (segment (start 143.51 59.69) (end 154.305 59.69) (width 0.25) (layer "F.Cu") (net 7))
 (segment (start 145.96 112.94) (end 145.96 111.296396) (width 0.25) (layer "F.Cu") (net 7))
 (segment (start 143.61 110.66) (end 142.24 109.29) (width 0.25) (layer "F.Cu") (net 7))
 (segment (start 149.86 157.48) (end 149.86 116.84) (width 0.25) (layer "F.Cu") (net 7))
 (segment (start 149.86 116.84) (end 145.96 112.94) (width 0.25) (layer "F.Cu") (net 7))
 (segment (start 165.5175 50.165) (end 166.38 51.0275) (width 0.25) (layer "F.Cu") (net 7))
 (segment (start 140.97 69.8) (end 141.416396 69.8) (width 0.25) (layer "F.Cu") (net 7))
 (segment (start 145.323604 110.66) (end 143.61 110.66) (width 0.25) (layer "F.Cu") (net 7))
 (segment (start 154.94 53.34) (end 158.115 50.165) (width 0.25) (layer "F.Cu") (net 7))
 (segment (start 142.875 60.325) (end 143.51 59.69) (width 0.25) (layer "F.Cu") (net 7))
 (segment (start 141.416396 69.8) (end 142.875 68.341396) (width 0.25) (layer "F.Cu") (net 7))
 (segment (start 142.24 109.29) (end 142.24 71.07) (width 0.25) (layer "F.Cu") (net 7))
 (segment (start 148.73 158.89) (end 147.32 157.48) (width 0.25) (layer "F.Cu") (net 4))
 (segment (start 137.16 51.0775) (end 136.793 51.0775) (width 0.25) (layer "F.Cu") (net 4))
 (segment (start 142.24 68.34) (end 142.24 63.45) (width 0.25) (layer "F.Cu") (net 4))
 (segment (start 137.16 106.68) (end 137.16 68.58) (width 0.25) (layer "F.Cu") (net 4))
 (segment (start 136.793 51.0775) (end 135.255 52.6155) (width 0.25) (layer "F.Cu") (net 4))
 (segment (start 135.255 60.96) (end 139.75 60.96) (width 0.25) (layer "F.Cu") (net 4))
 (segment (start 137.16 68.58) (end 142 68.58) (width 0.25) (layer "F.Cu") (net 4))
 (segment (start 147.32 157.48) (end 147.32 116.84) (width 0.25) (layer "F.Cu") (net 4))
 (segment (start 139.75 60.96) (end 140.97 62.18) (width 0.25) (layer "F.Cu") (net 4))
 (segment (start 147.32 116.84) (end 137.16 106.68) (width 0.25) (layer "F.Cu") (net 4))
 (segment (start 142 68.58) (end 142.24 68.34) (width 0.25) (layer "F.Cu") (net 4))
 (segment (start 142.24 63.45) (end 140.97 62.18) (width 0.25) (layer "F.Cu") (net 4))
 (segment (start 148.73 163.936025) (end 148.73 158.89) (width 0.25) (layer "F.Cu") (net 4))
 (via (at 135.255 60.96) (size 0.8) (drill 0.4) (layers "F.Cu" "B.Cu") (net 4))
 (via (at 135.255 52.6155) (size 0.8) (drill 0.4) (layers "F.Cu" "B.Cu") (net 4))
 (segment (start 135.255 52.6155) (end 135.255 60.96) (width 0.25) (layer "B.Cu") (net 4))
 (segment (start 134.62 106.68) (end 134.62 68.58) (width 0.25) (layer "F.Cu") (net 6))
 (segment (start 135.94 67.26) (end 140.97 67.26) (width 0.25) (layer "F.Cu") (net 6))
 (segment (start 144.78 157.48) (end 144.78 116.84) (width 0.25) (layer "F.Cu") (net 6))
 (segment (start 145.88 163.936025) (end 145.88 158.58) (width 0.25) (layer "F.Cu") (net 6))
 (segment (start 145.88 158.58) (end 144.78 157.48) (width 0.25) (layer "F.Cu") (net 6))
 (segment (start 134.62 68.58) (end 135.94 67.26) (width 0.25) (layer "F.Cu") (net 6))
 (segment (start 144.78 116.84) (end 134.62 106.68) (width 0.25) (layer "F.Cu") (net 6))
 (segment (start 132.08 66.04) (end 133.4 64.72) (width 0.25) (layer "F.Cu") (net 5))
 (segment (start 132.08 106.68) (end 132.08 66.04) (width 0.25) (layer "F.Cu") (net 5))
 (segment (start 142.93 163.936025) (end 142.93 117.53) (width 0.25) (layer "F.Cu") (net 5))
 (segment (start 133.4 64.72) (end 140.97 64.72) (width 0.25) (layer "F.Cu") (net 5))
 (segment (start 142.93 117.53) (end 132.08 106.68) (width 0.25) (layer "F.Cu") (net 5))
 (segment (start 131.445 53.34) (end 139.75 53.34) (width 0.25) (layer "F.Cu") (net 1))
 (segment (start 139.75 53.34) (end 140.97 54.56) (width 0.25) (layer "F.Cu") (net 1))
 (segment (start 131.445 55.88) (end 139.75 55.88) (width 0.25) (layer "F.Cu") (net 2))
 (segment (start 139.75 55.88) (end 140.97 57.1) (width 0.25) (layer "F.Cu") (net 2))
 (segment (start 160.665 51.0775) (end 161.725 52.1375) (width 0.25) (layer "F.Cu") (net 34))
 (segment (start 160.36 69.8) (end 158.75 69.8) (width 0.25) (layer "F.Cu") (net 34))
 (segment (start 161.725 68.435) (end 160.36 69.8) (width 0.25) (layer "F.Cu") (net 34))
 (segment (start 161.725 52.1375) (end 161.725 68.435) (width 0.25) (layer "F.Cu") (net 34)))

